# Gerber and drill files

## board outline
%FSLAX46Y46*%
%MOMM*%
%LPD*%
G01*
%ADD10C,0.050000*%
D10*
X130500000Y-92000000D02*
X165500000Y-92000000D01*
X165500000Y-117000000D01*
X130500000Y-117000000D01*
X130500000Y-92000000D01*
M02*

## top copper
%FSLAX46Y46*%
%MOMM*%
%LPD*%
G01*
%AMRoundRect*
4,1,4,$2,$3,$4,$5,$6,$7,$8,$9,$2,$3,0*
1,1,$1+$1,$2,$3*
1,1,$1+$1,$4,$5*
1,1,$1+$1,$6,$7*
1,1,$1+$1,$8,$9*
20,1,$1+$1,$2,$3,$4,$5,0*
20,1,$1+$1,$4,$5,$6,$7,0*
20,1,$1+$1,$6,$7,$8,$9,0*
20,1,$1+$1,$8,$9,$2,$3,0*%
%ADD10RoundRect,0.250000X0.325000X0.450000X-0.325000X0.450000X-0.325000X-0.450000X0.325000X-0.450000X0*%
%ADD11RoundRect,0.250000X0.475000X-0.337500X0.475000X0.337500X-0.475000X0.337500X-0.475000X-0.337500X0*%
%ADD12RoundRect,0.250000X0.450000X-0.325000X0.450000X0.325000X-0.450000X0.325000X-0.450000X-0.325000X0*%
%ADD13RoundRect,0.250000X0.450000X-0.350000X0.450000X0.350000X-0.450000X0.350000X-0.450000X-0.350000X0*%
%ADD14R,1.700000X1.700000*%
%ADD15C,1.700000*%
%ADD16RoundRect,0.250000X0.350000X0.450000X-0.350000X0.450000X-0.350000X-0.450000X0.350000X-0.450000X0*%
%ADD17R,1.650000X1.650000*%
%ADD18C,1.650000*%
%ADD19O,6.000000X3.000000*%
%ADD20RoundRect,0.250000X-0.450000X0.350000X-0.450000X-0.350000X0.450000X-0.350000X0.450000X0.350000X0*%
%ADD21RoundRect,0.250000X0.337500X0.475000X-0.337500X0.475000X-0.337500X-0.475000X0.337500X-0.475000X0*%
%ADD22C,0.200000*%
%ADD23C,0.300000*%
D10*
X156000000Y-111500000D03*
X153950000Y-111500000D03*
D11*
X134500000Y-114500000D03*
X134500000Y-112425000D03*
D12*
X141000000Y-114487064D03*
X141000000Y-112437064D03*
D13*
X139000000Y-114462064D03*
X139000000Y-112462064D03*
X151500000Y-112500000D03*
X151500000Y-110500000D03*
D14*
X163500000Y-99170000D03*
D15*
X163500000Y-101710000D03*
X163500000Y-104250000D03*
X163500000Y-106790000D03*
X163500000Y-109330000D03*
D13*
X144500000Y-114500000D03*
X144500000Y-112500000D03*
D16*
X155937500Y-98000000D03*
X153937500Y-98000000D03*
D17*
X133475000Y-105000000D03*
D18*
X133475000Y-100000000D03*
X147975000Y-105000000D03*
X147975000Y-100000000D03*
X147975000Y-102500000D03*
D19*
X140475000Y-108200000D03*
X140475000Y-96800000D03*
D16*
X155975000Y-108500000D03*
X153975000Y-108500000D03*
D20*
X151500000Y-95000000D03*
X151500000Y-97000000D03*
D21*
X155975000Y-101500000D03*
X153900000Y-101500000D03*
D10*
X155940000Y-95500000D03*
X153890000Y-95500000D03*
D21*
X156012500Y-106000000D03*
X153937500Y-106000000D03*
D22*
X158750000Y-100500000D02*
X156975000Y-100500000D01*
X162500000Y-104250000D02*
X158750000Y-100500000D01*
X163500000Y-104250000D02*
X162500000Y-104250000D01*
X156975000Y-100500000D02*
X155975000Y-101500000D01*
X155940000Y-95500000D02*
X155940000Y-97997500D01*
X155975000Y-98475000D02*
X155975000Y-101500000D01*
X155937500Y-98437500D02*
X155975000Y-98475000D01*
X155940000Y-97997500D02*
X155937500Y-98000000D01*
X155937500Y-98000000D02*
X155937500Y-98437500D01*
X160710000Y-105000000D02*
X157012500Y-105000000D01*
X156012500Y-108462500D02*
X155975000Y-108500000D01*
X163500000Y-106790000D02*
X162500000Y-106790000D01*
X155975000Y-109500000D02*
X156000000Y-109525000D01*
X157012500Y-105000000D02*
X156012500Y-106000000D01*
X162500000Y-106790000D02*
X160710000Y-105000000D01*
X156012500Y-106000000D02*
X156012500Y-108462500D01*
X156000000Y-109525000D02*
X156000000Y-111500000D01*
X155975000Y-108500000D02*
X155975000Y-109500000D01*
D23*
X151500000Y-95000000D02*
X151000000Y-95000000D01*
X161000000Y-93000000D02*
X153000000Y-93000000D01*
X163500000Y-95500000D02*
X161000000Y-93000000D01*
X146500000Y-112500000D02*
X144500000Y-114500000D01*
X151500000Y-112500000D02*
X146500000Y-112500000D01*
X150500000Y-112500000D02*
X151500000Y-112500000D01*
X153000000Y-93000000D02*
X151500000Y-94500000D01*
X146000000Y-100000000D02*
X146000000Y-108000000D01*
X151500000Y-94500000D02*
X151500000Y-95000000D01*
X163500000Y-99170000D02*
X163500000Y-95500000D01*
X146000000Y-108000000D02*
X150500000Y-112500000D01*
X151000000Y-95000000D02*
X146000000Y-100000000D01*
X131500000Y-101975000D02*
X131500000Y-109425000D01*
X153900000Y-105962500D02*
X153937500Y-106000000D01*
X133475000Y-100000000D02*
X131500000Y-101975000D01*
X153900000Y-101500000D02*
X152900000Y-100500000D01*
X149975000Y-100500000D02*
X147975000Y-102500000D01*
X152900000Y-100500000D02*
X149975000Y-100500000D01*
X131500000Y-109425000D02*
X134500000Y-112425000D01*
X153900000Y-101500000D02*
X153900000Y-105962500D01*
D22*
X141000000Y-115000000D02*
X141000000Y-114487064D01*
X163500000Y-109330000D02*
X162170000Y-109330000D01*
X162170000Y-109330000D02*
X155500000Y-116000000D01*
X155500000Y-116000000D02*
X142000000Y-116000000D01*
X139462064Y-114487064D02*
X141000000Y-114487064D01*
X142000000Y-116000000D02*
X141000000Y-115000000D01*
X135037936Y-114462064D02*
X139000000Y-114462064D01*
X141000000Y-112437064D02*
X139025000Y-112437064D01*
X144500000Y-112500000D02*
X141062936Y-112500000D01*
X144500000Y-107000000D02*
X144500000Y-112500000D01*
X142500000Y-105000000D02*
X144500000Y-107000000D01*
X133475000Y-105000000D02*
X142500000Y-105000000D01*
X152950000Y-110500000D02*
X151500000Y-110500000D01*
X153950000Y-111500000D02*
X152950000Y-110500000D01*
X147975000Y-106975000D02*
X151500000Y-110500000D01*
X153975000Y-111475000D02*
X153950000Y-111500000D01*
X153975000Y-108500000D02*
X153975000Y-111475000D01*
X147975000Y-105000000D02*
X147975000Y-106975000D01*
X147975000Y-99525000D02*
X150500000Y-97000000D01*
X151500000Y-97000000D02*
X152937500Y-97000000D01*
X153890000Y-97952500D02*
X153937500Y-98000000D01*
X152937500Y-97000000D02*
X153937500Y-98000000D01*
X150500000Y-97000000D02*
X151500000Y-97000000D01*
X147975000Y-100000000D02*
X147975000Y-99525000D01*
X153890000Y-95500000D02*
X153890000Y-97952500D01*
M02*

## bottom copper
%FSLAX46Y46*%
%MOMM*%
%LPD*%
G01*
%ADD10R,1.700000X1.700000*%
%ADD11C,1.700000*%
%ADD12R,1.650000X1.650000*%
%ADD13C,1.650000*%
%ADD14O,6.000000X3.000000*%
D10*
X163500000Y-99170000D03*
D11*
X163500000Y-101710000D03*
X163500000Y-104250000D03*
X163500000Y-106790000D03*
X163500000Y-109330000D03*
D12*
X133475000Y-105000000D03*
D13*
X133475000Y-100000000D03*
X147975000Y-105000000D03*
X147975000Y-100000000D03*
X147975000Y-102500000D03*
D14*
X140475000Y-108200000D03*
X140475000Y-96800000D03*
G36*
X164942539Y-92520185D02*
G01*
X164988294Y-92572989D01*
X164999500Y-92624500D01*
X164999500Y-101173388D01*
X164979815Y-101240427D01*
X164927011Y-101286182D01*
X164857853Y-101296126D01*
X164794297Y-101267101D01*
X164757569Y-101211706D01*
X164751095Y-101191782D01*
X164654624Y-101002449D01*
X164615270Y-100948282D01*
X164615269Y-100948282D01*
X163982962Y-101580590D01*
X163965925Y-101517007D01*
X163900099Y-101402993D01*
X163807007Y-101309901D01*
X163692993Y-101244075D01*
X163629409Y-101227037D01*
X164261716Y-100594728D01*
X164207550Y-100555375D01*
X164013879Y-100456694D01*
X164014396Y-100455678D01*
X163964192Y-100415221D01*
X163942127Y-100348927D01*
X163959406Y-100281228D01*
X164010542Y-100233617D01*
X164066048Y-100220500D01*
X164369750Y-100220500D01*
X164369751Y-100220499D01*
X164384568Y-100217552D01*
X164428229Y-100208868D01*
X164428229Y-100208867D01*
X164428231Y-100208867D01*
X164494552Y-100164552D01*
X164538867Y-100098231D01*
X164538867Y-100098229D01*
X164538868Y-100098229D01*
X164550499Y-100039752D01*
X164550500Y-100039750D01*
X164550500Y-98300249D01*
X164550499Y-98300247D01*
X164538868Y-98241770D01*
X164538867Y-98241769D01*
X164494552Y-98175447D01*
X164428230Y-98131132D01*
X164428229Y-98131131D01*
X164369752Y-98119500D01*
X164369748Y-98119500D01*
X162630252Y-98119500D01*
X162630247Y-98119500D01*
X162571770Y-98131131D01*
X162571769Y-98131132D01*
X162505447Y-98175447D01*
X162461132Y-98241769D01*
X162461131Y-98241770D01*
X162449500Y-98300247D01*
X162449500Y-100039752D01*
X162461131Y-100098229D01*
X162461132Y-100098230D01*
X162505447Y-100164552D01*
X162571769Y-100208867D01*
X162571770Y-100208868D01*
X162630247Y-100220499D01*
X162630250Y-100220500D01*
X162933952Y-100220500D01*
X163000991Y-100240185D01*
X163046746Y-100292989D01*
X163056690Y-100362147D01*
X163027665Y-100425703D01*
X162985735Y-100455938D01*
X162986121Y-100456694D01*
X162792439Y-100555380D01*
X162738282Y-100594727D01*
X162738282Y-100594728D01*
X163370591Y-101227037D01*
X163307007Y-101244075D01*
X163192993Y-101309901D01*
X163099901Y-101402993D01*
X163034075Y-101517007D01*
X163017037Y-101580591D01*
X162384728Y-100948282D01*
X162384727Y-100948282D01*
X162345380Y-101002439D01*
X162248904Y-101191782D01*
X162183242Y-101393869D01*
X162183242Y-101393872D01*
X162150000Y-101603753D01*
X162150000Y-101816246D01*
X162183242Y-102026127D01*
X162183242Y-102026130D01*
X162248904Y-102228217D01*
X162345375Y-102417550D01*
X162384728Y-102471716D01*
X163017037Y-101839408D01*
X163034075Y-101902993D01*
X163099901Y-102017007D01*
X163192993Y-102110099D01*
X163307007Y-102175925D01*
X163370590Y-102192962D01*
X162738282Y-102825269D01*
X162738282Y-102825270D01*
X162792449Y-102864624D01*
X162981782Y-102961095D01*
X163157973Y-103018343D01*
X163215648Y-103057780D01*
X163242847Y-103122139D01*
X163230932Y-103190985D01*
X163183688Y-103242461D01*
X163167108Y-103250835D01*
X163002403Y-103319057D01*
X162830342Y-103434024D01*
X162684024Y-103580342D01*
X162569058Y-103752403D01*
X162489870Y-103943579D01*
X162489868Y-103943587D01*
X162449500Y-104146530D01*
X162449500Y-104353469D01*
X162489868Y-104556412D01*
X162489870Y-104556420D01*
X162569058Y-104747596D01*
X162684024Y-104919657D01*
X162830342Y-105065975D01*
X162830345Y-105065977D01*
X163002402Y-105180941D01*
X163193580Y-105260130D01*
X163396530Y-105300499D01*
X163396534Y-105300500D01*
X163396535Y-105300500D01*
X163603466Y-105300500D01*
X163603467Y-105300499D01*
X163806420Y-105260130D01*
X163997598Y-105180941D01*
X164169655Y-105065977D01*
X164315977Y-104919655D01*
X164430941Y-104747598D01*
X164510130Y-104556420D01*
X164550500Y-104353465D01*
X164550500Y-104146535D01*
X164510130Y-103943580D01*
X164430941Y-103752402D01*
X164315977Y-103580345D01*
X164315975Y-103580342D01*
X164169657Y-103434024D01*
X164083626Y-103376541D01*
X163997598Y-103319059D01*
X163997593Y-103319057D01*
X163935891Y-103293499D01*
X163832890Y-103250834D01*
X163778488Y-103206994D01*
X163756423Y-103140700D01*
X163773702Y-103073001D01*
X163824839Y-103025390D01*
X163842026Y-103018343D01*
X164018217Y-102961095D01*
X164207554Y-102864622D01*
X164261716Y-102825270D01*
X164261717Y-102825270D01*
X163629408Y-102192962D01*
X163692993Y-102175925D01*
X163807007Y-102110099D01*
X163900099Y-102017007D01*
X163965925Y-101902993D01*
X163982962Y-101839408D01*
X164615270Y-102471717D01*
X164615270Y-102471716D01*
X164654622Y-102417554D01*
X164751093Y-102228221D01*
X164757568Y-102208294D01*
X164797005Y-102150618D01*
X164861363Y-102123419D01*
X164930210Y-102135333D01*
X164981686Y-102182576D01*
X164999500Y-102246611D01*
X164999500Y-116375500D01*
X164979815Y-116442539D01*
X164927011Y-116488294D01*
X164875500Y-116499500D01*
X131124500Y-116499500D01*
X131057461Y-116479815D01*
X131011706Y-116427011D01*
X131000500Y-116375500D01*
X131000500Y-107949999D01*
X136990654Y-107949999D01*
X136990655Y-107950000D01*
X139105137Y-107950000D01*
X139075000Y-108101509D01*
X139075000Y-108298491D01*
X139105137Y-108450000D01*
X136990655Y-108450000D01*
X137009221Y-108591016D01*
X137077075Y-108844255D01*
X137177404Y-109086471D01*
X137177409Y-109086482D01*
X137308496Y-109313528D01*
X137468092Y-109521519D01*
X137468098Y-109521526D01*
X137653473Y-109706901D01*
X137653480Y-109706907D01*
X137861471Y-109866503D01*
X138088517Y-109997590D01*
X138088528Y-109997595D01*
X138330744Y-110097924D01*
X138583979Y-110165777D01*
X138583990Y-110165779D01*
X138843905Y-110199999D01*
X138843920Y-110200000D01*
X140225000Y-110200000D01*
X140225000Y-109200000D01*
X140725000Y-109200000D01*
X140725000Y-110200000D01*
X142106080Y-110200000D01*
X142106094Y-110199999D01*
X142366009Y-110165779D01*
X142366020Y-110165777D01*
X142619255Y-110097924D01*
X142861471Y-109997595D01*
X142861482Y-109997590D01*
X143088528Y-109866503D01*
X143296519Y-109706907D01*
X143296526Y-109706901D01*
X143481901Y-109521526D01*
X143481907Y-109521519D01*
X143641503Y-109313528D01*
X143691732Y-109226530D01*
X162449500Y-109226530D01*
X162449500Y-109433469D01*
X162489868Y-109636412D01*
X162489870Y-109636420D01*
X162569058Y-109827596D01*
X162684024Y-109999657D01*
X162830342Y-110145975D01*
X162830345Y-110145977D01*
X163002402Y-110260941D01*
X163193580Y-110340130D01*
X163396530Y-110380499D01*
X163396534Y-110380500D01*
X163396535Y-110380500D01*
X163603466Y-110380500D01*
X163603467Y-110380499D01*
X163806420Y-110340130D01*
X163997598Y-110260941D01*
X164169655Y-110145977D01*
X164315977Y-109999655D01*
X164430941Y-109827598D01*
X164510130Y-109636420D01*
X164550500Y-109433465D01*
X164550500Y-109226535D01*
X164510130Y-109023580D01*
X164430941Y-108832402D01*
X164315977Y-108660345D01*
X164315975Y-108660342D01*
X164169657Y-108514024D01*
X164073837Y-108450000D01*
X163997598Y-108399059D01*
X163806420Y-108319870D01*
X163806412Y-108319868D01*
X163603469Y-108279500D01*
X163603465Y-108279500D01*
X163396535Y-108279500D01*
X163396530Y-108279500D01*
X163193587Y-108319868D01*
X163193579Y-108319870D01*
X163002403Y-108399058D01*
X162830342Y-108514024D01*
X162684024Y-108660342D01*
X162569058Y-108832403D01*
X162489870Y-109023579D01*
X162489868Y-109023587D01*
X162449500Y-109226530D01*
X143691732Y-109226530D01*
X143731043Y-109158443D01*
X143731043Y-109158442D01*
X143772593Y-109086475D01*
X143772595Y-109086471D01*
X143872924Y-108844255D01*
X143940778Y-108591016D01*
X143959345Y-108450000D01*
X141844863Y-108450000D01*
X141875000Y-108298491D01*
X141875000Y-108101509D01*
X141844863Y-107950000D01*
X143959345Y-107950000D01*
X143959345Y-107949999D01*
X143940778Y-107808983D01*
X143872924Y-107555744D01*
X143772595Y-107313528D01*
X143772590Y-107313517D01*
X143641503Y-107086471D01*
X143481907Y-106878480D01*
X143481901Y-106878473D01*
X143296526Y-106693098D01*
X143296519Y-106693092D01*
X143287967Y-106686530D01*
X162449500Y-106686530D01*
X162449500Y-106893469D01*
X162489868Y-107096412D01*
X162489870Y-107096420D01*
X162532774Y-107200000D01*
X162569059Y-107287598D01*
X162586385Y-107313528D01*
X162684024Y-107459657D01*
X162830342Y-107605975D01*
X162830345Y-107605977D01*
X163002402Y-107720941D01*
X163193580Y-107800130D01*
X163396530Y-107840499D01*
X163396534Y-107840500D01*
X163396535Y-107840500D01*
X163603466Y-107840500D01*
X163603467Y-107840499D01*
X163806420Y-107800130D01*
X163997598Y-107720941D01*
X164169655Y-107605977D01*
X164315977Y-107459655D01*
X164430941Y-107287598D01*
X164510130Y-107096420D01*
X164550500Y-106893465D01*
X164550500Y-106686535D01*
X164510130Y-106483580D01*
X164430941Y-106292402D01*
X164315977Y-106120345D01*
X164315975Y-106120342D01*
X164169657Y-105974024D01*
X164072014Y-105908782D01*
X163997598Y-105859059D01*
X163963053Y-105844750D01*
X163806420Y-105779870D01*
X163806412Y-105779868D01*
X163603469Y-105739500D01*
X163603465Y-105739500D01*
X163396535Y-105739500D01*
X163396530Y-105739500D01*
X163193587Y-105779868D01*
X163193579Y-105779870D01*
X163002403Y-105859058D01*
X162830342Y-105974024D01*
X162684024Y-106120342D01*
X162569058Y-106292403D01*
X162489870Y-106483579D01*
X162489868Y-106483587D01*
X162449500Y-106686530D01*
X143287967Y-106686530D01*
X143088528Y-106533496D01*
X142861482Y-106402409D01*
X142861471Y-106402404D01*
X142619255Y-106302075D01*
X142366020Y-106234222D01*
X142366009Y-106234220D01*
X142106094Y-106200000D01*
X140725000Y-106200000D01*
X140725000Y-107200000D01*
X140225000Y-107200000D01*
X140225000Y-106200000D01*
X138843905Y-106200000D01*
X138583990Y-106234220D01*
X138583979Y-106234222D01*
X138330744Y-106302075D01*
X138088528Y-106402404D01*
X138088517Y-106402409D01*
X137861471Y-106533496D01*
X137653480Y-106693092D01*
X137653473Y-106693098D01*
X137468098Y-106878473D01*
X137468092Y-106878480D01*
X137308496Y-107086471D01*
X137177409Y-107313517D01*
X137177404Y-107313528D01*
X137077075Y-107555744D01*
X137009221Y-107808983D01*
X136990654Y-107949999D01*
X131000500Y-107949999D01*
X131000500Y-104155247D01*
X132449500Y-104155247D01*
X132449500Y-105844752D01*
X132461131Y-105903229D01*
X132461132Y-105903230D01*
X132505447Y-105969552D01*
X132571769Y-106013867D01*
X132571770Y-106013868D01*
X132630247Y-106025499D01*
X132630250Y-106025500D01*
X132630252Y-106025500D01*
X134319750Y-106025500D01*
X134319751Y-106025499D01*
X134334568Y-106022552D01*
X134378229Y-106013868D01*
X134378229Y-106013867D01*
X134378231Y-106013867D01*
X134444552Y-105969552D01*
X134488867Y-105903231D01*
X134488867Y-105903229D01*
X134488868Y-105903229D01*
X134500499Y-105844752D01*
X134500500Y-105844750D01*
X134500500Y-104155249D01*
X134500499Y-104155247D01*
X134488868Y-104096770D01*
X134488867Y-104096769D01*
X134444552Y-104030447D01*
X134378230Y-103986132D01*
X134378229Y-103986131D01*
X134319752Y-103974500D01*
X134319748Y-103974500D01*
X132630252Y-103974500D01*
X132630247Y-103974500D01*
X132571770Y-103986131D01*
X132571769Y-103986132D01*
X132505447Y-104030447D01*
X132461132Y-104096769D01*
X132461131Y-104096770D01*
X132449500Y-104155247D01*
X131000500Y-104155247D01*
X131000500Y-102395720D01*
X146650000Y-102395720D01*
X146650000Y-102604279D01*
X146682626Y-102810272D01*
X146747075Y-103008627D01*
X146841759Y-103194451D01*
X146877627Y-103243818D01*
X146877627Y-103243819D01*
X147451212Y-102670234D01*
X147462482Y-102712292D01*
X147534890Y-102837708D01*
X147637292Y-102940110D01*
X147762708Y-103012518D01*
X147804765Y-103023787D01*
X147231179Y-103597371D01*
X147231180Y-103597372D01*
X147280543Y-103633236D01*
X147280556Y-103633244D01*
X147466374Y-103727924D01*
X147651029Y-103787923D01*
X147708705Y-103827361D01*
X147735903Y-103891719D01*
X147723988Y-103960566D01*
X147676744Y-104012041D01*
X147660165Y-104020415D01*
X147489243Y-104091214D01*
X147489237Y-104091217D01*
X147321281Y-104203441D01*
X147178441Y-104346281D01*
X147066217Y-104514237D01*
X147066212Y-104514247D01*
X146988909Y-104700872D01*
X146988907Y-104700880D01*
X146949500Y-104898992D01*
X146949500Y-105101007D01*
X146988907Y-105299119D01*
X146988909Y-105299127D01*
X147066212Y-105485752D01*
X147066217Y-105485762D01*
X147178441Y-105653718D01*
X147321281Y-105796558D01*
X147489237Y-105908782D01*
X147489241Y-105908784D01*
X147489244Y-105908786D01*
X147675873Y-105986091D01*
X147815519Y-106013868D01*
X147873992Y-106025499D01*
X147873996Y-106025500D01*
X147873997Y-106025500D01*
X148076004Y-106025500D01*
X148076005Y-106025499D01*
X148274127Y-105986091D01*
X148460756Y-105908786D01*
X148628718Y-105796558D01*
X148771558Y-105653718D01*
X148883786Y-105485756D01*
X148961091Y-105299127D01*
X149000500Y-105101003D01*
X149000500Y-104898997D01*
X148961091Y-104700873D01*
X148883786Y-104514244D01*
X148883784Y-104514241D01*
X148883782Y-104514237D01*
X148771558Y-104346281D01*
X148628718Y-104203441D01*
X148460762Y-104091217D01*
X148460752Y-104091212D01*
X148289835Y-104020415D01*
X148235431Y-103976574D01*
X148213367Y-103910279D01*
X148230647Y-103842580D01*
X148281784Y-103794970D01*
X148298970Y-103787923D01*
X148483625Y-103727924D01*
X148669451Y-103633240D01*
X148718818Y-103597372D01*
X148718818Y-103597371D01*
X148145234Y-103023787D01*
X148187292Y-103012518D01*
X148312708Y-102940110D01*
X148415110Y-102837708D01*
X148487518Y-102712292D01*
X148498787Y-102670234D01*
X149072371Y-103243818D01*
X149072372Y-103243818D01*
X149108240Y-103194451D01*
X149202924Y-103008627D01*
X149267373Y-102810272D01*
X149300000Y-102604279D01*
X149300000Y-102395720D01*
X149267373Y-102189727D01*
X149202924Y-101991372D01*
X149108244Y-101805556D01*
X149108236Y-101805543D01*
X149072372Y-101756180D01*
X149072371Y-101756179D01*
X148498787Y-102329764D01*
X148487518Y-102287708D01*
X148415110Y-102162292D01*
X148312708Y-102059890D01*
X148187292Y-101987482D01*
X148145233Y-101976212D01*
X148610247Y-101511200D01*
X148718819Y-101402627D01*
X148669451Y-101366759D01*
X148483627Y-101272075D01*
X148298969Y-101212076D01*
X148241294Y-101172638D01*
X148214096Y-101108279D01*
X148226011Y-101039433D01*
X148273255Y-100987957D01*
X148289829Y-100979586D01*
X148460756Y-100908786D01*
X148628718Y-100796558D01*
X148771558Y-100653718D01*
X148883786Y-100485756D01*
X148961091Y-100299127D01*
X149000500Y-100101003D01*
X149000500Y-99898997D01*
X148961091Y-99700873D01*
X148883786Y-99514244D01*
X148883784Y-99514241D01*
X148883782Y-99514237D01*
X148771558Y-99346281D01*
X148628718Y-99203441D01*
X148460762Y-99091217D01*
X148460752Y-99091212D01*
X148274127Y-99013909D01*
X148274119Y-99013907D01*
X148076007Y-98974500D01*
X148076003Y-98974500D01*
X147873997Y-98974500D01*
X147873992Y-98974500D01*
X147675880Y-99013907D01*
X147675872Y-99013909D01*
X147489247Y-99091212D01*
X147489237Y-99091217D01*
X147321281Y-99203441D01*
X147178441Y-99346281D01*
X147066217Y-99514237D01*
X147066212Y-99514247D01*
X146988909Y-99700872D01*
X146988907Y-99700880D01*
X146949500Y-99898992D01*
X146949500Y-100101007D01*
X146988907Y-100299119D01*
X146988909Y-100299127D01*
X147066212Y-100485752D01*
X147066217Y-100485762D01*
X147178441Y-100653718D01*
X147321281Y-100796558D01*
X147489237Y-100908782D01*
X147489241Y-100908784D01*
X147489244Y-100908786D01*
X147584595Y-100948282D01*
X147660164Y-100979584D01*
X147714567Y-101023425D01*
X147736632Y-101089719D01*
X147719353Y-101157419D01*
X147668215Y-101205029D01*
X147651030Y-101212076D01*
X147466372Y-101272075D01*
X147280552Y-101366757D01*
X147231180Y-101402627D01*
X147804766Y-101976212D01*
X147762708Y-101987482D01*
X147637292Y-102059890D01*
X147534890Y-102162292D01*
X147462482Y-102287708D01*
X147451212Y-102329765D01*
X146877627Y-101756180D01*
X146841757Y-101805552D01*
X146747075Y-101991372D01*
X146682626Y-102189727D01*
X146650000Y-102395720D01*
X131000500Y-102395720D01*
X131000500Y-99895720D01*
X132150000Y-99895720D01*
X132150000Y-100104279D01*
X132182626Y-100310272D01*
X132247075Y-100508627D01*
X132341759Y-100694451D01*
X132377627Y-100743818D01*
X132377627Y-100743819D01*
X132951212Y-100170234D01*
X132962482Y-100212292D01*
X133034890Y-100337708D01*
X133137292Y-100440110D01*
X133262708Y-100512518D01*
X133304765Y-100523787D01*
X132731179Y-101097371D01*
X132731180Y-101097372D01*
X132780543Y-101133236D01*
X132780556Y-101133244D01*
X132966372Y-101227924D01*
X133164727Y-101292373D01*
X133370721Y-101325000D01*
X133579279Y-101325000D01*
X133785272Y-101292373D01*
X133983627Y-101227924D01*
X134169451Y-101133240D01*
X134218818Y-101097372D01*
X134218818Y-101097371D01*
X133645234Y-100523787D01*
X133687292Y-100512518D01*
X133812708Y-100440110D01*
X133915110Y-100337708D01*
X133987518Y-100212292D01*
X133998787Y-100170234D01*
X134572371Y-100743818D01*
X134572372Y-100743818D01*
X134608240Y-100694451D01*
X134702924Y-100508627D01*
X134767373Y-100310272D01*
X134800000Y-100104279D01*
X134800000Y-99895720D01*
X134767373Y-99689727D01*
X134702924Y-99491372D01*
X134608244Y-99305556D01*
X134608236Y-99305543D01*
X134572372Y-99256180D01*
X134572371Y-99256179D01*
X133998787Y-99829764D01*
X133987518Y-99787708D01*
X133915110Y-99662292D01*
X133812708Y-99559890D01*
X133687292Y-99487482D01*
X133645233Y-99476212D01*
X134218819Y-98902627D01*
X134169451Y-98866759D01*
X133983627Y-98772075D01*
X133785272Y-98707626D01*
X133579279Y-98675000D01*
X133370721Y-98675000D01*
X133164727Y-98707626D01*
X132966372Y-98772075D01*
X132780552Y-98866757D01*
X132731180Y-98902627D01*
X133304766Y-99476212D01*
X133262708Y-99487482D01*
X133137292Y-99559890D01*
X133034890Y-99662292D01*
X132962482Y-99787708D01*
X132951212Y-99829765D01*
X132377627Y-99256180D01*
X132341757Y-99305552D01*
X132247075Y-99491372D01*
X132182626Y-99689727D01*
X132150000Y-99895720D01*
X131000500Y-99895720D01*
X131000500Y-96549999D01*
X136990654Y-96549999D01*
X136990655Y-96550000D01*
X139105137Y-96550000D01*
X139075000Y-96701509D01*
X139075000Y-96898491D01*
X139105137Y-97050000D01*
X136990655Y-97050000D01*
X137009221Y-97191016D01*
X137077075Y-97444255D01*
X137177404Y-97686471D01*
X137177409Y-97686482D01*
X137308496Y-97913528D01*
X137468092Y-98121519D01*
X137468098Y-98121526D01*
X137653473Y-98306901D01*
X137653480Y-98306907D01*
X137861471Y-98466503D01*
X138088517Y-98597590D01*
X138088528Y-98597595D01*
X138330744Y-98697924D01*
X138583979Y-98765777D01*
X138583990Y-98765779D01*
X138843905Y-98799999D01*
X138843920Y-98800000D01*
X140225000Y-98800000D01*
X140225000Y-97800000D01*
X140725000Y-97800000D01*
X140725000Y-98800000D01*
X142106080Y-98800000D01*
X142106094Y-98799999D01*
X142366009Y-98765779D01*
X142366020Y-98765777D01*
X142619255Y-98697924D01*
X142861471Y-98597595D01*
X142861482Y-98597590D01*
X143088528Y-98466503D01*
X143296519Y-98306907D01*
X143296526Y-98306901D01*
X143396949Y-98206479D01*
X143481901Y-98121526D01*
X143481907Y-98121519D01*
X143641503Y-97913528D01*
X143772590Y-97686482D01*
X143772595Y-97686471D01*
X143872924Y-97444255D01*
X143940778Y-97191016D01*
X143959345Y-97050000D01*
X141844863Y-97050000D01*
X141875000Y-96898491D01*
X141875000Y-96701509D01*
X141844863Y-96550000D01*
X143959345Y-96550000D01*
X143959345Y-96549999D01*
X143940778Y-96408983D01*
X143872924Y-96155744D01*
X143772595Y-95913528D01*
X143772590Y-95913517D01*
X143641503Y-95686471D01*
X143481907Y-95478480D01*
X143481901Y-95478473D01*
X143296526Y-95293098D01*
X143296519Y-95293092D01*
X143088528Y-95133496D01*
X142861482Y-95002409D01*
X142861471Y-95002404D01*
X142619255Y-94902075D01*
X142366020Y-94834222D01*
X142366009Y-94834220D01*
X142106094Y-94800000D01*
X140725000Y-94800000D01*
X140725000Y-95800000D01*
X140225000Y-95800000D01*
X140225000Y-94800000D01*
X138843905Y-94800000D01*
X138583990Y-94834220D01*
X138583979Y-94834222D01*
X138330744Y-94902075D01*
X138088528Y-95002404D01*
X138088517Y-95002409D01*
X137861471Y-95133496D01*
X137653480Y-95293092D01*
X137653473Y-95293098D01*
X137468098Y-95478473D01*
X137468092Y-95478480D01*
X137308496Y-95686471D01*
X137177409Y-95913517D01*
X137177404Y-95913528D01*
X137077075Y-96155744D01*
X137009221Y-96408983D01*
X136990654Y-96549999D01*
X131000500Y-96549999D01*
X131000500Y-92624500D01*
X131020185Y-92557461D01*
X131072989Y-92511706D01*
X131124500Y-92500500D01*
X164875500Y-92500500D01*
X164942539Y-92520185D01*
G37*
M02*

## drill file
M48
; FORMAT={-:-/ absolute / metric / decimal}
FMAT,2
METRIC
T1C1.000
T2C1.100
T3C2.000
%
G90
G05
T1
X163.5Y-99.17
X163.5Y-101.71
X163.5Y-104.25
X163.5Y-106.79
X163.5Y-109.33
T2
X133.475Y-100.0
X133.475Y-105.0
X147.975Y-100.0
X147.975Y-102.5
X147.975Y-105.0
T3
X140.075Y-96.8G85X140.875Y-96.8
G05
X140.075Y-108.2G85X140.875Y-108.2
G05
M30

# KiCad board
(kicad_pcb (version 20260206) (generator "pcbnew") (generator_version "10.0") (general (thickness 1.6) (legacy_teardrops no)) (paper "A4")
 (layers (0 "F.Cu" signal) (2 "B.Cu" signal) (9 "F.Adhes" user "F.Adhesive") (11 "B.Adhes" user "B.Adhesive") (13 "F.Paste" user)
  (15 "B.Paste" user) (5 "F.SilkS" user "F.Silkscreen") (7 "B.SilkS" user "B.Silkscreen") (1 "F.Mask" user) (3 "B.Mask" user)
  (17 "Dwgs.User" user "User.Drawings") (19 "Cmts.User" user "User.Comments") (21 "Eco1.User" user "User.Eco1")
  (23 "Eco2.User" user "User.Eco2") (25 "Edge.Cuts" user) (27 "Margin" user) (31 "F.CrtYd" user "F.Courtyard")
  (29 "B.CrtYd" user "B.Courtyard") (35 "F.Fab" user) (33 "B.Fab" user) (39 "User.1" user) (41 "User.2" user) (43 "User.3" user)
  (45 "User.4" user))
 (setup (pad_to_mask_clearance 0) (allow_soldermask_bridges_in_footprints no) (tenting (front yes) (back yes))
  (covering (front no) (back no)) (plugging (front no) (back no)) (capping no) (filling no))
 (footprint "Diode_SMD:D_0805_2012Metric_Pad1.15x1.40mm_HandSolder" (layer "F.Cu") (at 154.975 111.5 180)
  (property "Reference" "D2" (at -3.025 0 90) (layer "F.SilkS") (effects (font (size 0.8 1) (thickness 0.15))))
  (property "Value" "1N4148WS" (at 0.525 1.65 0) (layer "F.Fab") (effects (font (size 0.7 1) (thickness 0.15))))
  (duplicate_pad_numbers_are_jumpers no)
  (pad "1" smd roundrect (at -1.025 0 180) (size 1.15 1.4) (layers "F.Cu" "F.Mask" "F.Paste") (roundrect_rratio 0.217391) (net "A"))
  (pad "2" smd roundrect (at 1.025 0 180) (size 1.15 1.4) (layers "F.Cu" "F.Mask" "F.Paste") (roundrect_rratio 0.217391) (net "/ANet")))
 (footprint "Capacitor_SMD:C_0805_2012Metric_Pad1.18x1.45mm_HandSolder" (layer "F.Cu") (at 134.5 113.4625 90)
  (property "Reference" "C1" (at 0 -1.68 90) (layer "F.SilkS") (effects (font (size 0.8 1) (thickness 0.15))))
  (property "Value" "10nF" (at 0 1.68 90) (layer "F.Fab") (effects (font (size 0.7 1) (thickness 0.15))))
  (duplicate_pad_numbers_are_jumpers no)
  (pad "1" smd roundrect (at -1.0375 0 90) (size 1.175 1.45) (layers "F.Cu" "F.Mask" "F.Paste") (roundrect_rratio 0.212766) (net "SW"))
  (pad "2" smd roundrect (at 1.0375 0 90) (size 1.175 1.45) (layers "F.Cu" "F.Mask" "F.Paste") (roundrect_rratio 0.212766) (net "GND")))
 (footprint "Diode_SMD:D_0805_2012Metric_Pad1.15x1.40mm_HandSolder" (layer "F.Cu") (at 141 113.462064 90)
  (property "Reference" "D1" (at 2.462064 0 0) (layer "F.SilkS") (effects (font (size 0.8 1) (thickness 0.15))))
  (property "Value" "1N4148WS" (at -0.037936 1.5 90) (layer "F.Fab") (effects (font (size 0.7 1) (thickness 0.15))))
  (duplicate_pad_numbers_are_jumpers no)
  (pad "1" smd roundrect (at -1.025 0 90) (size 1.15 1.4) (layers "F.Cu" "F.Mask" "F.Paste") (roundrect_rratio 0.217391) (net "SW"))
  (pad "2" smd roundrect (at 1.025 0 90) (size 1.15 1.4) (layers "F.Cu" "F.Mask" "F.Paste") (roundrect_rratio 0.217391) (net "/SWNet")))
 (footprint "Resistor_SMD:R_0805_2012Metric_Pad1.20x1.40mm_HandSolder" (layer "F.Cu") (at 139 113.462064 90)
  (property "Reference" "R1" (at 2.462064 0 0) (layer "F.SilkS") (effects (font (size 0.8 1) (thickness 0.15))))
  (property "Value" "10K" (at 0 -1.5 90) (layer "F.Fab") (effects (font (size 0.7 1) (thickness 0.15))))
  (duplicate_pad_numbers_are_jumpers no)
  (pad "1" smd roundrect (at -1 0 90) (size 1.2 1.4) (layers "F.Cu" "F.Mask" "F.Paste") (roundrect_rratio 0.208333) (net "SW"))
  (pad "2" smd roundrect (at 1 0 90) (size 1.2 1.4) (layers "F.Cu" "F.Mask" "F.Paste") (roundrect_rratio 0.208333) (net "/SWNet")))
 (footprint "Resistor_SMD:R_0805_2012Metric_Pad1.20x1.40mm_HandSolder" (layer "F.Cu") (at 151.5 111.5 90)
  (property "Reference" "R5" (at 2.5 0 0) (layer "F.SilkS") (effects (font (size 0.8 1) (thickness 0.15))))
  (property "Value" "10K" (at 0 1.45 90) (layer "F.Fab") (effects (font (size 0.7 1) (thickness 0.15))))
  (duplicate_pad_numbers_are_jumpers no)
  (pad "1" smd roundrect (at -1 0 90) (size 1.2 1.4) (layers "F.Cu" "F.Mask" "F.Paste") (roundrect_rratio 0.208333) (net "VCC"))
  (pad "2" smd roundrect (at 1 0 90) (size 1.2 1.4) (layers "F.Cu" "F.Mask" "F.Paste") (roundrect_rratio 0.208333) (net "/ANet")))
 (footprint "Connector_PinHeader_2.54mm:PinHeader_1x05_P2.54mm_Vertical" (layer "F.Cu") (at 163.5 99.17)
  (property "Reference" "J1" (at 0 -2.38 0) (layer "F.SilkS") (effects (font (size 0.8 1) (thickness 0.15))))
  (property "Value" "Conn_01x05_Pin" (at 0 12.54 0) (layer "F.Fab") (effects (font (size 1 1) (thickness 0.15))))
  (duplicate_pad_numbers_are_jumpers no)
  (pad "1" thru_hole rect (at 0 0) (size 1.7 1.7) (drill 1) (layers "*.Cu" "*.Mask") (remove_unused_layers no) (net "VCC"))
  (pad "2" thru_hole circle (at 0 2.54) (size 1.7 1.7) (drill 1) (layers "*.Cu" "*.Mask") (remove_unused_layers no) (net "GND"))
  (pad "3" thru_hole circle (at 0 5.08) (size 1.7 1.7) (drill 1) (layers "*.Cu" "*.Mask") (remove_unused_layers no) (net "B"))
  (pad "4" thru_hole circle (at 0 7.62) (size 1.7 1.7) (drill 1) (layers "*.Cu" "*.Mask") (remove_unused_layers no) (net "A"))
  (pad "5" thru_hole circle (at 0 10.16) (size 1.7 1.7) (drill 1) (layers "*.Cu" "*.Mask") (remove_unused_layers no) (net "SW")))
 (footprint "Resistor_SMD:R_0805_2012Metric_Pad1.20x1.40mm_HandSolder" (layer "F.Cu") (at 144.5 113.5 90)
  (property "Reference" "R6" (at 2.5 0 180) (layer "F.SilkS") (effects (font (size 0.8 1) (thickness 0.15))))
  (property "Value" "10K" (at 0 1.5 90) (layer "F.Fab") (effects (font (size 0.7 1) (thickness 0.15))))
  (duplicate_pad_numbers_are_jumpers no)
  (pad "1" smd roundrect (at -1 0 90) (size 1.2 1.4) (layers "F.Cu" "F.Mask" "F.Paste") (roundrect_rratio 0.208333) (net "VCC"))
  (pad "2" smd roundrect (at 1 0 90) (size 1.2 1.4) (layers "F.Cu" "F.Mask" "F.Paste") (roundrect_rratio 0.208333) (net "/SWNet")))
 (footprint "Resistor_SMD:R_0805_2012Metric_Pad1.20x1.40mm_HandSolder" (layer "F.Cu") (at 154.9375 98 180)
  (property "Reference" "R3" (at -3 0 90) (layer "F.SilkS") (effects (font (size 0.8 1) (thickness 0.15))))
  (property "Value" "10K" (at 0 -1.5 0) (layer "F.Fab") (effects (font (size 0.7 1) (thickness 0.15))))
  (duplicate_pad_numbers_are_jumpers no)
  (pad "1" smd roundrect (at -1 0 180) (size 1.2 1.4) (layers "F.Cu" "F.Mask" "F.Paste") (roundrect_rratio 0.208333) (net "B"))
  (pad "2" smd roundrect (at 1 0 180) (size 1.2 1.4) (layers "F.Cu" "F.Mask" "F.Paste") (roundrect_rratio 0.208333) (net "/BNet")))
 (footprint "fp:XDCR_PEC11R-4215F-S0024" (layer "F.Cu") (at 140.475 102.5 90)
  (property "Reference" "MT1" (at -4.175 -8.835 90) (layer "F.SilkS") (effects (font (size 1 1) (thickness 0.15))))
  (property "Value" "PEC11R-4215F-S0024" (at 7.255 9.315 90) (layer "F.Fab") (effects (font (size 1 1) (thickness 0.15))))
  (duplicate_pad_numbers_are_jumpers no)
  (pad "1" thru_hole rect (at -2.5 -7 90) (size 1.65 1.65) (drill 1.1) (layers "*.Cu" "*.Mask") (remove_unused_layers no) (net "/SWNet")
   (solder_mask_margin 0.102))
  (pad "2" thru_hole circle (at 2.5 -7 90) (size 1.65 1.65) (drill 1.1) (layers "*.Cu" "*.Mask") (remove_unused_layers no) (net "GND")
   (solder_mask_margin 0.102))
  (pad "A" thru_hole circle (at -2.5 7.5 90) (size 1.65 1.65) (drill 1.1) (layers "*.Cu" "*.Mask") (remove_unused_layers no) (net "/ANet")
   (solder_mask_margin 0.102))
  (pad "B" thru_hole circle (at 2.5 7.5 90) (size 1.65 1.65) (drill 1.1) (layers "*.Cu" "*.Mask") (remove_unused_layers no) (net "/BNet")
   (solder_mask_margin 0.102))
  (pad "COM" thru_hole circle (at 0 7.5 90) (size 1.65 1.65) (drill 1.1) (layers "*.Cu" "*.Mask") (remove_unused_layers no) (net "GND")
   (solder_mask_margin 0.102))
  (pad "S1" thru_hole oval (at -5.7 0 90) (size 3 6) (drill oval 2 2.8) (layers "*.Cu" "*.Mask") (remove_unused_layers no) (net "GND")
   (solder_mask_margin 0.102))
  (pad "S2" thru_hole oval (at 5.7 0 90) (size 3 6) (drill oval 2 2.8) (layers "*.Cu" "*.Mask") (remove_unused_layers no) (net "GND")
   (solder_mask_margin 0.102)))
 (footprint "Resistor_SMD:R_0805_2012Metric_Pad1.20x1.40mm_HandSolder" (layer "F.Cu") (at 154.975 108.5 180)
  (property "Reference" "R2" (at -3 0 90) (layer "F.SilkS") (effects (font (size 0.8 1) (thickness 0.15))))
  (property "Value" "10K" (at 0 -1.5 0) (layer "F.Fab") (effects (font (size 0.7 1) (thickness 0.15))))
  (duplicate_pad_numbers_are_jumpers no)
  (pad "1" smd roundrect (at -1 0 180) (size 1.2 1.4) (layers "F.Cu" "F.Mask" "F.Paste") (roundrect_rratio 0.208333) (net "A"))
  (pad "2" smd roundrect (at 1 0 180) (size 1.2 1.4) (layers "F.Cu" "F.Mask" "F.Paste") (roundrect_rratio 0.208333) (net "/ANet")))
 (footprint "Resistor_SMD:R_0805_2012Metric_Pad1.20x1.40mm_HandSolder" (layer "F.Cu") (at 151.5 96 -90)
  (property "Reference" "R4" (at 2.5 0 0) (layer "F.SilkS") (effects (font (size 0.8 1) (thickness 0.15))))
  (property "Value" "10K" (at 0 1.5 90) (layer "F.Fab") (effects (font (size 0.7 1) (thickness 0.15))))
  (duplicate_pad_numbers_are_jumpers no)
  (pad "1" smd roundrect (at -1 0 270) (size 1.2 1.4) (layers "F.Cu" "F.Mask" "F.Paste") (roundrect_rratio 0.208333) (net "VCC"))
  (pad "2" smd roundrect (at 1 0 270) (size 1.2 1.4) (layers "F.Cu" "F.Mask" "F.Paste") (roundrect_rratio 0.208333) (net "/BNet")))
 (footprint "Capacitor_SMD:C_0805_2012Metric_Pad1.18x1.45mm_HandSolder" (layer "F.Cu") (at 154.9375 101.5 180)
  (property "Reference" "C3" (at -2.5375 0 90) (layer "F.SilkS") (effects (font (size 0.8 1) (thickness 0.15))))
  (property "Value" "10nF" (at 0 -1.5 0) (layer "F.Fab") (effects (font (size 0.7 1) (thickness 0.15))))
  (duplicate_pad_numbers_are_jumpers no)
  (pad "1" smd roundrect (at -1.0375 0 180) (size 1.175 1.45) (layers "F.Cu" "F.Mask" "F.Paste") (roundrect_rratio 0.212766) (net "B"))
  (pad "2" smd roundrect (at 1.0375 0 180) (size 1.175 1.45) (layers "F.Cu" "F.Mask" "F.Paste") (roundrect_rratio 0.212766) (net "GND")))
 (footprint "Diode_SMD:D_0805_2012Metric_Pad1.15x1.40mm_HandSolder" (layer "F.Cu") (at 154.915 95.5 180)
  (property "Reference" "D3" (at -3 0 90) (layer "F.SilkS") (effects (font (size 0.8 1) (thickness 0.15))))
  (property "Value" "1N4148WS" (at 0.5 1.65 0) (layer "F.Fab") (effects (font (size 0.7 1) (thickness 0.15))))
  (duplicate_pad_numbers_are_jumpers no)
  (pad "1" smd roundrect (at -1.025 0 180) (size 1.15 1.4) (layers "F.Cu" "F.Mask" "F.Paste") (roundrect_rratio 0.217391) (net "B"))
  (pad "2" smd roundrect (at 1.025 0 180) (size 1.15 1.4) (layers "F.Cu" "F.Mask" "F.Paste") (roundrect_rratio 0.217391) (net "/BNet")))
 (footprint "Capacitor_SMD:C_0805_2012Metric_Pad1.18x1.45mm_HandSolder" (layer "F.Cu") (at 154.975 106 180)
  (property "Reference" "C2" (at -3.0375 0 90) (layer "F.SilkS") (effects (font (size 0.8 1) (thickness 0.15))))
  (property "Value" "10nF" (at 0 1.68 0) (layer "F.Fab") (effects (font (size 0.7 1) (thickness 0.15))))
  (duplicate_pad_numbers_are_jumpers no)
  (pad "1" smd roundrect (at -1.0375 0 180) (size 1.175 1.45) (layers "F.Cu" "F.Mask" "F.Paste") (roundrect_rratio 0.212766) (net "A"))
  (pad "2" smd roundrect (at 1.0375 0 180) (size 1.175 1.45) (layers "F.Cu" "F.Mask" "F.Paste") (roundrect_rratio 0.212766) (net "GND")))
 (gr_rect (start 130.5 92) (end 165.5 117) (stroke (width 0.05) (type solid)) (fill no) (layer "Edge.Cuts"))
 (segment (start 158.75 100.5) (end 156.975 100.5) (width 0.2) (layer "F.Cu") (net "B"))
 (segment (start 162.5 104.25) (end 158.75 100.5) (width 0.2) (layer "F.Cu") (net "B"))
 (segment (start 163.5 104.25) (end 162.5 104.25) (width 0.2) (layer "F.Cu") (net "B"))
 (segment (start 156.975 100.5) (end 155.975 101.5) (width 0.2) (layer "F.Cu") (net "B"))
 (segment (start 155.94 95.5) (end 155.94 97.9975) (width 0.2) (layer "F.Cu") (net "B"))
 (segment (start 155.975 98.475) (end 155.975 101.5) (width 0.2) (layer "F.Cu") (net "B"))
 (segment (start 155.9375 98.4375) (end 155.975 98.475) (width 0.2) (layer "F.Cu") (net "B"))
 (segment (start 155.94 97.9975) (end 155.9375 98) (width 0.2) (layer "F.Cu") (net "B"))
 (segment (start 155.9375 98) (end 155.9375 98.4375) (width 0.2) (layer "F.Cu") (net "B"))
 (segment (start 160.71 105) (end 157.0125 105) (width 0.2) (layer "F.Cu") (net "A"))
 (segment (start 156.0125 108.4625) (end 155.975 108.5) (width 0.2) (layer "F.Cu") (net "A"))
 (segment (start 163.5 106.79) (end 162.5 106.79) (width 0.2) (layer "F.Cu") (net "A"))
 (segment (start 155.975 109.5) (end 156 109.525) (width 0.2) (layer "F.Cu") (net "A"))
 (segment (start 157.0125 105) (end 156.0125 106) (width 0.2) (layer "F.Cu") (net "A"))
 (segment (start 162.5 106.79) (end 160.71 105) (width 0.2) (layer "F.Cu") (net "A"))
 (segment (start 156.0125 106) (end 156.0125 108.4625) (width 0.2) (layer "F.Cu") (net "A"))
 (segment (start 156 109.525) (end 156 111.5) (width 0.2) (layer "F.Cu") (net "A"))
 (segment (start 155.975 108.5) (end 155.975 109.5) (width 0.2) (layer "F.Cu") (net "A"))
 (segment (start 151.5 95) (end 151 95) (width 0.3) (layer "F.Cu") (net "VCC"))
 (segment (start 161 93) (end 153 93) (width 0.3) (layer "F.Cu") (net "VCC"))
 (segment (start 163.5 95.5) (end 161 93) (width 0.3) (layer "F.Cu") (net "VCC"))
 (segment (start 146.5 112.5) (end 144.5 114.5) (width 0.3) (layer "F.Cu") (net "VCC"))
 (segment (start 151.5 112.5) (end 146.5 112.5) (width 0.3) (layer "F.Cu") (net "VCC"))
 (segment (start 150.5 112.5) (end 151.5 112.5) (width 0.3) (layer "F.Cu") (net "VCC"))
 (segment (start 153 93) (end 151.5 94.5) (width 0.3) (layer "F.Cu") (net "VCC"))
 (segment (start 146 100) (end 146 108) (width 0.3) (layer "F.Cu") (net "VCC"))
 (segment (start 151.5 94.5) (end 151.5 95) (width 0.3) (layer "F.Cu") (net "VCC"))
 (segment (start 163.5 99.17) (end 163.5 95.5) (width 0.3) (layer "F.Cu") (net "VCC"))
 (segment (start 146 108) (end 150.5 112.5) (width 0.3) (layer "F.Cu") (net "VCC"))
 (segment (start 151 95) (end 146 100) (width 0.3) (layer "F.Cu") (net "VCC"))
 (segment (start 131.5 101.975) (end 131.5 109.425) (width 0.3) (layer "F.Cu") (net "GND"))
 (segment (start 153.9 105.9625) (end 153.9375 106) (width 0.3) (layer "F.Cu") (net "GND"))
 (segment (start 133.475 100) (end 131.5 101.975) (width 0.3) (layer "F.Cu") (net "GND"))
 (segment (start 153.9 101.5) (end 152.9 100.5) (width 0.3) (layer "F.Cu") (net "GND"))
 (segment (start 149.975 100.5) (end 147.975 102.5) (width 0.3) (layer "F.Cu") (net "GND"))
 (segment (start 152.9 100.5) (end 149.975 100.5) (width 0.3) (layer "F.Cu") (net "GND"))
 (segment (start 131.5 109.425) (end 134.5 112.425) (width 0.3) (layer "F.Cu") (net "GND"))
 (segment (start 153.9 101.5) (end 153.9 105.9625) (width 0.3) (layer "F.Cu") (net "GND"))
 (segment (start 141 115) (end 141 114.487064) (width 0.2) (layer "F.Cu") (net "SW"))
 (segment (start 163.5 109.33) (end 162.17 109.33) (width 0.2) (layer "F.Cu") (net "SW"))
 (segment (start 162.17 109.33) (end 155.5 116) (width 0.2) (layer "F.Cu") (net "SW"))
 (segment (start 155.5 116) (end 142 116) (width 0.2) (layer "F.Cu") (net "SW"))
 (segment (start 139.462064 114.487064) (end 141 114.487064) (width 0.2) (layer "F.Cu") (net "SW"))
 (segment (start 142 116) (end 141 115) (width 0.2) (layer "F.Cu") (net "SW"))
 (segment (start 135.037936 114.462064) (end 139 114.462064) (width 0.2) (layer "F.Cu") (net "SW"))
 (segment (start 141 112.437064) (end 139.025 112.437064) (width 0.2) (layer "F.Cu") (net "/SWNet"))
 (segment (start 144.5 112.5) (end 141.062936 112.5) (width 0.2) (layer "F.Cu") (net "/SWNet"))
 (segment (start 144.5 107) (end 144.5 112.5) (width 0.2) (layer "F.Cu") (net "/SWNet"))
 (segment (start 142.5 105) (end 144.5 107) (width 0.2) (layer "F.Cu") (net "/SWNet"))
 (segment (start 133.475 105) (end 142.5 105) (width 0.2) (layer "F.Cu") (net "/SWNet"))
 (segment (start 152.95 110.5) (end 151.5 110.5) (width 0.2) (layer "F.Cu") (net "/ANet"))
 (segment (start 153.95 111.5) (end 152.95 110.5) (width 0.2) (layer "F.Cu") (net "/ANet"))
 (segment (start 147.975 106.975) (end 151.5 110.5) (width 0.2) (layer "F.Cu") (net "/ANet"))
 (segment (start 153.975 111.475) (end 153.95 111.5) (width 0.2) (layer "F.Cu") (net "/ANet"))
 (segment (start 153.975 108.5) (end 153.975 111.475) (width 0.2) (layer "F.Cu") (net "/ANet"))
 (segment (start 147.975 105) (end 147.975 106.975) (width 0.2) (layer "F.Cu") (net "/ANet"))
 (segment (start 147.975 99.525) (end 150.5 97) (width 0.2) (layer "F.Cu") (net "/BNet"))
 (segment (start 151.5 97) (end 152.9375 97) (width 0.2) (layer "F.Cu") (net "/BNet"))
 (segment (start 153.89 97.9525) (end 153.9375 98) (width 0.2) (layer "F.Cu") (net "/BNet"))
 (segment (start 152.9375 97) (end 153.9375 98) (width 0.2) (layer "F.Cu") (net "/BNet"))
 (segment (start 150.5 97) (end 151.5 97) (width 0.2) (layer "F.Cu") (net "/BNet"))
 (segment (start 147.975 100) (end 147.975 99.525) (width 0.2) (layer "F.Cu") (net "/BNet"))
 (segment (start 153.89 95.5) (end 153.89 97.9525) (width 0.2) (layer "F.Cu") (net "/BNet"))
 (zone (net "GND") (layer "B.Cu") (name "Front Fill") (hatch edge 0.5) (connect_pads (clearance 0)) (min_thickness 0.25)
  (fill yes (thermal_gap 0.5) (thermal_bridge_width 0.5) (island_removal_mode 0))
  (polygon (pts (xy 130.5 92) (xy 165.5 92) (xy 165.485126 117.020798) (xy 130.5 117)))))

